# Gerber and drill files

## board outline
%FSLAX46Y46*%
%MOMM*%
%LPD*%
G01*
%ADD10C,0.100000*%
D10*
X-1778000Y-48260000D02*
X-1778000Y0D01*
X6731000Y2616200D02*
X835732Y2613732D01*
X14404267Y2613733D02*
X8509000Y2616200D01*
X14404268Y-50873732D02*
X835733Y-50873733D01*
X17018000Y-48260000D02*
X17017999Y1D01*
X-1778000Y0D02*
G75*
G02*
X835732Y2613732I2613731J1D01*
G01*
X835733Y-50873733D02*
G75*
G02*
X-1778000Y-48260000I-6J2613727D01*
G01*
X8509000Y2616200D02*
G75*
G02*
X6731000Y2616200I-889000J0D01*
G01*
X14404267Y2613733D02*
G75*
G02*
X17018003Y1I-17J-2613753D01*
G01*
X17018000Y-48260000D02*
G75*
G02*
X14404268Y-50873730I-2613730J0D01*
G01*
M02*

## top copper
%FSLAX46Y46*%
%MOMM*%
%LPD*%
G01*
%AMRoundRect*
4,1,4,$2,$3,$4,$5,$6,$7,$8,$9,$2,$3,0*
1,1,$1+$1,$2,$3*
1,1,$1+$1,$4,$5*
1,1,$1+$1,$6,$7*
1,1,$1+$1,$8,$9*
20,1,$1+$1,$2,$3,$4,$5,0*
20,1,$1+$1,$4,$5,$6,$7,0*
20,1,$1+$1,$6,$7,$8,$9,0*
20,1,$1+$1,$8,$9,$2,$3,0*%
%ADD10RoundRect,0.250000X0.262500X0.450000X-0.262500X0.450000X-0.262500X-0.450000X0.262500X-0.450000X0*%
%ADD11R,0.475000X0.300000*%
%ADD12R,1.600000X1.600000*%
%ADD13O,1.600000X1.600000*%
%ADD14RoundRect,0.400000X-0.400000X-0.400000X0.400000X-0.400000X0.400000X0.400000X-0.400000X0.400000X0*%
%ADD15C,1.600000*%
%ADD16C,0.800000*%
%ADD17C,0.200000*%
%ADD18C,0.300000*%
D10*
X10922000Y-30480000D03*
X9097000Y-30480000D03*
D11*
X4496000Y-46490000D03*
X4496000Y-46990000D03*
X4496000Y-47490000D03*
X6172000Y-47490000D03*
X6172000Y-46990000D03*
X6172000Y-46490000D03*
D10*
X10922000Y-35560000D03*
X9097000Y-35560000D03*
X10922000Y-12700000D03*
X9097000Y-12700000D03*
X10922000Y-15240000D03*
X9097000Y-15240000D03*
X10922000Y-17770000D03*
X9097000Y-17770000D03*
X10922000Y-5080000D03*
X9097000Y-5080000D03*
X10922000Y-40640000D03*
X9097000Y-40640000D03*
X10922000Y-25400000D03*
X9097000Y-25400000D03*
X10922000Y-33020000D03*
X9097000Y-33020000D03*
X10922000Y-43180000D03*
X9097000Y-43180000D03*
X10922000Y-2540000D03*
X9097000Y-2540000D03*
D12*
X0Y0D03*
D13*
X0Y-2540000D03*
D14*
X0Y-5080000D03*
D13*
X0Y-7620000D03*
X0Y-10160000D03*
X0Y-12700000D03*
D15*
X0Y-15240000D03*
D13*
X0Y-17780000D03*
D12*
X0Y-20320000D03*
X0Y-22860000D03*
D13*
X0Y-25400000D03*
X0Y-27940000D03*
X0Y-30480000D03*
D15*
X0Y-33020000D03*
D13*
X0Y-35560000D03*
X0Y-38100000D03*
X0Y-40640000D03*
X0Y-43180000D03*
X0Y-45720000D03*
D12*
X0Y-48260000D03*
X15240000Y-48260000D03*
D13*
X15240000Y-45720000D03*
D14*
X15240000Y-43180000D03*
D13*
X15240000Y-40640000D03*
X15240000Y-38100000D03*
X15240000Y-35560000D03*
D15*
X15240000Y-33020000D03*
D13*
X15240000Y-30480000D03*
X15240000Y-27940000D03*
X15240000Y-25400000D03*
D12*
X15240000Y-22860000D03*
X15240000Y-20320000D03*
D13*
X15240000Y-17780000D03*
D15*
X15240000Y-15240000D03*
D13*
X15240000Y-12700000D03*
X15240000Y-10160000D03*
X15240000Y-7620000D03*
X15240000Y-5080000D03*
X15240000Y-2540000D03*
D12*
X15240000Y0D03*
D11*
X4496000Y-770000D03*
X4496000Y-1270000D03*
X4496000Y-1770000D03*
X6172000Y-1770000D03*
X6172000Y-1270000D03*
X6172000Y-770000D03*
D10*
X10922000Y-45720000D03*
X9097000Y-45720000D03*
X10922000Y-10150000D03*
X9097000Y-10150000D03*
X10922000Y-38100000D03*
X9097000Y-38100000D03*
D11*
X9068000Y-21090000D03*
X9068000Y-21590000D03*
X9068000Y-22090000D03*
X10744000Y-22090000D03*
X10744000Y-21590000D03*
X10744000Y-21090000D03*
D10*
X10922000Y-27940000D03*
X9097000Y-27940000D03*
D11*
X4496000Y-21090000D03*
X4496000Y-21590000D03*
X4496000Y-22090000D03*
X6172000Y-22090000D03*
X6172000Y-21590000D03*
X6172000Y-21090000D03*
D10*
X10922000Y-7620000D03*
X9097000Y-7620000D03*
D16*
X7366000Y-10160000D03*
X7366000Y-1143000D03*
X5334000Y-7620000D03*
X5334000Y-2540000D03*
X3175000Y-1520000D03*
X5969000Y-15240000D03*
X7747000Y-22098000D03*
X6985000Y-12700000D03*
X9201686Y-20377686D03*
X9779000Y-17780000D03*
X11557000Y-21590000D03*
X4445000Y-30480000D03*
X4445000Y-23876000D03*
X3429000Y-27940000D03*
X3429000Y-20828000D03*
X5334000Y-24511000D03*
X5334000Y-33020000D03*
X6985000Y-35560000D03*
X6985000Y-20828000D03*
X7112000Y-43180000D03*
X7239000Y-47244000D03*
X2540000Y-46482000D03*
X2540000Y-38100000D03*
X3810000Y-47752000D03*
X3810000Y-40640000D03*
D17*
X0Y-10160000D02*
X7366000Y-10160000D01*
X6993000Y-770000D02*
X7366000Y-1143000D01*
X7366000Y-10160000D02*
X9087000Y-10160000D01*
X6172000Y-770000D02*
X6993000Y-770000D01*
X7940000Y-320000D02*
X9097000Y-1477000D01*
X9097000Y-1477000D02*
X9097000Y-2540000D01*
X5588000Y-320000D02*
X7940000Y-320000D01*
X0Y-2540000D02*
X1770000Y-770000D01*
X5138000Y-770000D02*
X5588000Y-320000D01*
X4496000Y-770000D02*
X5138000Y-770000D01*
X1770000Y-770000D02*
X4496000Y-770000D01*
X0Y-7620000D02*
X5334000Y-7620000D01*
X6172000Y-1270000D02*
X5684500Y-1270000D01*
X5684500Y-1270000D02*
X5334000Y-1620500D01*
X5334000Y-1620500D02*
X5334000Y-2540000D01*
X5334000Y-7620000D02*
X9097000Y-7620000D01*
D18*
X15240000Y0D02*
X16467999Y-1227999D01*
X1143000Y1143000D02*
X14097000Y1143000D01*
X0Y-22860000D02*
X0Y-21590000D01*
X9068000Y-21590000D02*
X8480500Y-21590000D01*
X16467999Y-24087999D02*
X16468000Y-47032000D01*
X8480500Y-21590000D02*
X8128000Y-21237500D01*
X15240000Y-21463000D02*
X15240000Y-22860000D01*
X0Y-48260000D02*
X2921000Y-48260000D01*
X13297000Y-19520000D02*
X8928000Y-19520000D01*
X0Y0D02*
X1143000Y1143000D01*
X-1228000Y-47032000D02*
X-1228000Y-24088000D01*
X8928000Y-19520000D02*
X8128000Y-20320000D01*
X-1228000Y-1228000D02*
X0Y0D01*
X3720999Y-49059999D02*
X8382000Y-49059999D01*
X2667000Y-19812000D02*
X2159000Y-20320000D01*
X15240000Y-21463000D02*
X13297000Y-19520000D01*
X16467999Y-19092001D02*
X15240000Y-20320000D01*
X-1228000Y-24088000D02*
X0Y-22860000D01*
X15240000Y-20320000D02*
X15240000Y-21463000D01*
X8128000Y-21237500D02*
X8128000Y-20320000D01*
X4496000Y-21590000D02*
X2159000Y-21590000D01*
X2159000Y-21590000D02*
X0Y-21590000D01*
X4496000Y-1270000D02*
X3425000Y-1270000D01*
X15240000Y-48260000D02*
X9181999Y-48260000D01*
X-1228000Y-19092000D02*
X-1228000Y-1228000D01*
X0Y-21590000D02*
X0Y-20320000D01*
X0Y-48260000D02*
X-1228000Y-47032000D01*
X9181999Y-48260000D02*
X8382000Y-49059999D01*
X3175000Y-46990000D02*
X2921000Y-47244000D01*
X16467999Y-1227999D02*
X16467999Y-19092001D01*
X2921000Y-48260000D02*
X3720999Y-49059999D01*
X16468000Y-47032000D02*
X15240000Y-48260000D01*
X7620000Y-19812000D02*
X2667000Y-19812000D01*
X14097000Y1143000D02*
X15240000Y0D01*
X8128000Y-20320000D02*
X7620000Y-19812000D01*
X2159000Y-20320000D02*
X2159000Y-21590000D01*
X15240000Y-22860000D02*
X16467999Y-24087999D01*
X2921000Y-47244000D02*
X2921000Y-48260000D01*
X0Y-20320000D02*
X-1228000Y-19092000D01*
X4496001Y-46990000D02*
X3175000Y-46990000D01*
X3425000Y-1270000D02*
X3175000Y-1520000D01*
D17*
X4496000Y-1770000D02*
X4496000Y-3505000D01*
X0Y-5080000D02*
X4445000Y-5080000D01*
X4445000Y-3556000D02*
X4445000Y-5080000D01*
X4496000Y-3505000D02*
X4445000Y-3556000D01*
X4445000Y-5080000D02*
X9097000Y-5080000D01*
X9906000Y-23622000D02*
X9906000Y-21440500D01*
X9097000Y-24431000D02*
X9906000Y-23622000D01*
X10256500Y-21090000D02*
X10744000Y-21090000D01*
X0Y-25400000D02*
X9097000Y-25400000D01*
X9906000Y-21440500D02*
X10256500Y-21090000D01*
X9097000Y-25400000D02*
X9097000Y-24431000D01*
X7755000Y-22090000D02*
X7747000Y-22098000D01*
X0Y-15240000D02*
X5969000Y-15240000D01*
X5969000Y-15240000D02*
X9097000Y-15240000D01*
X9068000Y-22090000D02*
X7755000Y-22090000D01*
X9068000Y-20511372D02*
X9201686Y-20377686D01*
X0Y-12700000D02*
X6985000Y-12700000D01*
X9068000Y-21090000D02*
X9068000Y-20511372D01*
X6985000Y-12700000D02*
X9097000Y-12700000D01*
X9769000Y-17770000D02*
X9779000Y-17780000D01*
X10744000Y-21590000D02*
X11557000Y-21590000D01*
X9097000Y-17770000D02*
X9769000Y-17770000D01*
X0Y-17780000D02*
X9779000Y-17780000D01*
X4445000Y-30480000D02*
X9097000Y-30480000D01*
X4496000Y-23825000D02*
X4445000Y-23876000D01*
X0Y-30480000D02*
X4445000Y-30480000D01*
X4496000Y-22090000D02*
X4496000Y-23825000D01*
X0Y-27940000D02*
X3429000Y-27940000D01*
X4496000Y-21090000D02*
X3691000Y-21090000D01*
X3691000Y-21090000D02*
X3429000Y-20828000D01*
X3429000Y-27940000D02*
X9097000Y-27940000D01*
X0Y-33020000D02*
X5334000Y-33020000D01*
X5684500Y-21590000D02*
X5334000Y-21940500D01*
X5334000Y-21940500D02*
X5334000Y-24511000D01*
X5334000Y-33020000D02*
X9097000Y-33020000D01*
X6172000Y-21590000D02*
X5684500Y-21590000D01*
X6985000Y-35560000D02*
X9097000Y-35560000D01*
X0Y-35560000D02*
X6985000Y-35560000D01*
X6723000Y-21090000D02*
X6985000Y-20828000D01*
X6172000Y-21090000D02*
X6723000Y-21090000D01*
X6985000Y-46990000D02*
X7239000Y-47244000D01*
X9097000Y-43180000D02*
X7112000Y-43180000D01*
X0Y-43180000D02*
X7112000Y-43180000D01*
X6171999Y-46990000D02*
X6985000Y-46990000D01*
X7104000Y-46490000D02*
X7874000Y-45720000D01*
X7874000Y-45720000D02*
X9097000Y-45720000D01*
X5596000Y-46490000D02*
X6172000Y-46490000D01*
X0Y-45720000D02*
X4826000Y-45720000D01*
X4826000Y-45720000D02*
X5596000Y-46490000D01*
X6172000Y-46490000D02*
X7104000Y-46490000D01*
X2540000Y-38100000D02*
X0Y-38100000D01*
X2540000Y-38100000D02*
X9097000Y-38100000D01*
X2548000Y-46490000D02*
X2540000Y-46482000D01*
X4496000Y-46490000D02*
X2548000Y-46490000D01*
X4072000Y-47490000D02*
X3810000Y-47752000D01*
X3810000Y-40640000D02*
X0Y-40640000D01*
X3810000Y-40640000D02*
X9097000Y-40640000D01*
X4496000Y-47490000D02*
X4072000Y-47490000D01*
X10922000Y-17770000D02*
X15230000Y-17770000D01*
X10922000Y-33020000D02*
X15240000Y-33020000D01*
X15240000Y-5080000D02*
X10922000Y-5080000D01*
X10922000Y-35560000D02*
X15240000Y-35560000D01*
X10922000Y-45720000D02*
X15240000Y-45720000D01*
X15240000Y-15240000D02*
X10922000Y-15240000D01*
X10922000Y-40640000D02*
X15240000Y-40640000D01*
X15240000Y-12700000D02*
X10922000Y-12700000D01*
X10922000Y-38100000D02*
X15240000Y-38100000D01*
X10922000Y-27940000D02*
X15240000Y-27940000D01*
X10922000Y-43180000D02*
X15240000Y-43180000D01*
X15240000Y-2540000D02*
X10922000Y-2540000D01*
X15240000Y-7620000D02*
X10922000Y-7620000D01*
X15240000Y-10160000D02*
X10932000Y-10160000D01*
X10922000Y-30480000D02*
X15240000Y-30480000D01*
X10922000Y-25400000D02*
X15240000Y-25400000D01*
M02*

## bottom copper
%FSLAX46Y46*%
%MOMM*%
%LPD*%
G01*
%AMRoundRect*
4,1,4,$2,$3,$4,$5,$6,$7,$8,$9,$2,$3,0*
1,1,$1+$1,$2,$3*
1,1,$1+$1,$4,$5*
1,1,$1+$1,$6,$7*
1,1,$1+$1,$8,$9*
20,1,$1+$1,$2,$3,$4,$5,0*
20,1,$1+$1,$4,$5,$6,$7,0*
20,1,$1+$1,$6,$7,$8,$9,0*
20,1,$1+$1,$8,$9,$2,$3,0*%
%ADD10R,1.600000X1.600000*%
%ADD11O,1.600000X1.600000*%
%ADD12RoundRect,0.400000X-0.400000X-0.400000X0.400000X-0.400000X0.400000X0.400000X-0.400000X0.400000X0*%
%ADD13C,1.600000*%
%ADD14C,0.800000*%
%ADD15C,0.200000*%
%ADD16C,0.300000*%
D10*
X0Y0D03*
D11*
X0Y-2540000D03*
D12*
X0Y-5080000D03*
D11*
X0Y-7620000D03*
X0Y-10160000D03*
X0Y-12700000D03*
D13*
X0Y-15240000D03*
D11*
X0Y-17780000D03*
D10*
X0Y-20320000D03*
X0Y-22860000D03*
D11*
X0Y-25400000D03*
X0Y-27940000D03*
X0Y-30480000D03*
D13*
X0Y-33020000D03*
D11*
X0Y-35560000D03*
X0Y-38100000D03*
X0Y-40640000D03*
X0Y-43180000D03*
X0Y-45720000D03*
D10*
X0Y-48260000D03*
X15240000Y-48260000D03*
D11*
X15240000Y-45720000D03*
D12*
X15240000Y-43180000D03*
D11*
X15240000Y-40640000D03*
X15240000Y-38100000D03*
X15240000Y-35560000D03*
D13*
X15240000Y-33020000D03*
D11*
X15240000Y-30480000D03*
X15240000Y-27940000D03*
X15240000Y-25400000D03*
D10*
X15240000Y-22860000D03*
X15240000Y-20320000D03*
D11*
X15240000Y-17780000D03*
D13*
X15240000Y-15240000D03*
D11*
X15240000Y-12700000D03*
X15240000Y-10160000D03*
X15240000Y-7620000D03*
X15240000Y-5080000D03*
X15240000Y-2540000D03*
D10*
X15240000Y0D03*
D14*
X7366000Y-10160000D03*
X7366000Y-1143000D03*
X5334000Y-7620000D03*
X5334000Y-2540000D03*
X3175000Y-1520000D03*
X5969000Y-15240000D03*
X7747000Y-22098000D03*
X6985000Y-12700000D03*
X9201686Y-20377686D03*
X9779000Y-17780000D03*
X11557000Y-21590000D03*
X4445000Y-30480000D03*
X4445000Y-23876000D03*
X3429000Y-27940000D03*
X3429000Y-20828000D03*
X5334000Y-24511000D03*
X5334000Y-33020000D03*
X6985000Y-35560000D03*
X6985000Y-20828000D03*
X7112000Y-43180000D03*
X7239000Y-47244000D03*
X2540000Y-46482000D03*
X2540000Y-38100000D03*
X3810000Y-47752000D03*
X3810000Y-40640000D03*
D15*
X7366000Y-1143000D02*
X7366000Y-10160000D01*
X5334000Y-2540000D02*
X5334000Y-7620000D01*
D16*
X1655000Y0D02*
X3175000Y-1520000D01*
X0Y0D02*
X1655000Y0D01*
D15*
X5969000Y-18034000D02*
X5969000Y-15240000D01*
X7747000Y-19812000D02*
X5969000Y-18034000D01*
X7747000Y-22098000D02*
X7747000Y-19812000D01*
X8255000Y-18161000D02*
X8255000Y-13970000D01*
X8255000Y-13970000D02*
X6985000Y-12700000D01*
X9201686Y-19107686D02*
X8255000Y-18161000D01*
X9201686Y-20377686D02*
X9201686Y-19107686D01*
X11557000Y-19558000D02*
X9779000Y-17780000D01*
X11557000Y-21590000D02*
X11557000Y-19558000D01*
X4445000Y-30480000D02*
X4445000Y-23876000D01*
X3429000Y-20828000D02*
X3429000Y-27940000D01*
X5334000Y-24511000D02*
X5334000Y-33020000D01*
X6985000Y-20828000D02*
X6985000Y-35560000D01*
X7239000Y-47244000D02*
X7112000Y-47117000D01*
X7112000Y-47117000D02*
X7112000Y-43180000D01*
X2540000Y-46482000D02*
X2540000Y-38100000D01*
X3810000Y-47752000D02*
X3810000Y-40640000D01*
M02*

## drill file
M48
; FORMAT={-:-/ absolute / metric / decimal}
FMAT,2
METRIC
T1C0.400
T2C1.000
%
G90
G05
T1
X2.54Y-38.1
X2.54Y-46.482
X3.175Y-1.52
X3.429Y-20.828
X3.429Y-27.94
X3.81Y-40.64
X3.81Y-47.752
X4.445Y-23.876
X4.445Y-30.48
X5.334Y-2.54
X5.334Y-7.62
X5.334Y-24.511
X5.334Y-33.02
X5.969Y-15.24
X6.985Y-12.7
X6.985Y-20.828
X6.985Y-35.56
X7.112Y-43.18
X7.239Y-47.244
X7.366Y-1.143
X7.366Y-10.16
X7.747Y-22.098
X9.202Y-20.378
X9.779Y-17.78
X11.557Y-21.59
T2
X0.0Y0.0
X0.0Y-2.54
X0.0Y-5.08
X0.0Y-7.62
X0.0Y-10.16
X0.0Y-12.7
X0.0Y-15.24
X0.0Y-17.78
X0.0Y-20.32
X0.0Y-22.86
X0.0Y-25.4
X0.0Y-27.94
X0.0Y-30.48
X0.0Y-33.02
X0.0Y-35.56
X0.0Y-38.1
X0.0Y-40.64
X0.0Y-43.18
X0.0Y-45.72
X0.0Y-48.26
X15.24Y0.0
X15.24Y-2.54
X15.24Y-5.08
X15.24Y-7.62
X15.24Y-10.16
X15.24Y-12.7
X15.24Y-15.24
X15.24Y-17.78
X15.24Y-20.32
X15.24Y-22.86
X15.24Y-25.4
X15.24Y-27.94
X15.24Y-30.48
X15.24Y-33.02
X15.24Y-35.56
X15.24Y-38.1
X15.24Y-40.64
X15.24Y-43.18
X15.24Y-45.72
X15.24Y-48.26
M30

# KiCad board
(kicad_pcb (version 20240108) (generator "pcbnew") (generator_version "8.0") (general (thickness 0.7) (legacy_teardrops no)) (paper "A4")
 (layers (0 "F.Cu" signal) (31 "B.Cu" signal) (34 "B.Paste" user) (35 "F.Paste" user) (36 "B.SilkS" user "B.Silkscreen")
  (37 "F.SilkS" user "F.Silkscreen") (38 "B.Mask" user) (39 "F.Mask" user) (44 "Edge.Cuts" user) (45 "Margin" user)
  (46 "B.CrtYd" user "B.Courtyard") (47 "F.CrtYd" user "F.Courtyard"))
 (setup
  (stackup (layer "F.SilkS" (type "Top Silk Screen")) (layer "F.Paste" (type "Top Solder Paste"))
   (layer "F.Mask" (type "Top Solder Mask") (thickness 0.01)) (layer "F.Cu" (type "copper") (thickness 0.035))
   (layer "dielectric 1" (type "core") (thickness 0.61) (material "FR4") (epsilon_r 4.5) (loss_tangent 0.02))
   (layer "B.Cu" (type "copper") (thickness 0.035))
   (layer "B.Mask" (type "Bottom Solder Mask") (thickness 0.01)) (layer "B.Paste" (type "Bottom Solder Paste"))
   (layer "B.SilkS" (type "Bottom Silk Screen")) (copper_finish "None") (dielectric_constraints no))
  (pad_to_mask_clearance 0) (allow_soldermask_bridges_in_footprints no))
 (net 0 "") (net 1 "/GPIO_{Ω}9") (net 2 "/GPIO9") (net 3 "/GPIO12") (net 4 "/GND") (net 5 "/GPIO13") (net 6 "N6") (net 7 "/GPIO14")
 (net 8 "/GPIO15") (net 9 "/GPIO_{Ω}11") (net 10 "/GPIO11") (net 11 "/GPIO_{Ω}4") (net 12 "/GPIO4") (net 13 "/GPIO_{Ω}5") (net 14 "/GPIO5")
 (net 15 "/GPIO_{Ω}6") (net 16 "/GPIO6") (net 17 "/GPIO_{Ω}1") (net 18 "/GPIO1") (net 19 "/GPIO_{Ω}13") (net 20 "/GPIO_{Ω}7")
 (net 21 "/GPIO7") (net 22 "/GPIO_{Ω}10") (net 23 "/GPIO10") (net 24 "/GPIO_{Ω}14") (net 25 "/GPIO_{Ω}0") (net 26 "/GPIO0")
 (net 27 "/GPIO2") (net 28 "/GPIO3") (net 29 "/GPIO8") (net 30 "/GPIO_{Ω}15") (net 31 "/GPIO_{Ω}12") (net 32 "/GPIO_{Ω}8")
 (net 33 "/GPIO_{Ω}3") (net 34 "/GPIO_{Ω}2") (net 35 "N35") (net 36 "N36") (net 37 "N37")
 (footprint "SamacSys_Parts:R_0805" (layer "F.Cu") (at 10.0095 30.47 90)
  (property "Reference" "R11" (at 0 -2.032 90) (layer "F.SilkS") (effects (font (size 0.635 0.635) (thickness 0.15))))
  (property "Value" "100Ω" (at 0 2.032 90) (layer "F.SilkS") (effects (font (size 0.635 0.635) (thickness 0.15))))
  (pad "1" smd roundrect (at -0.01 0.9125 180) (size 1.025 1.4) (layers "F.Cu" "F.Paste" "F.Mask") (roundrect_rratio 0.243902)
   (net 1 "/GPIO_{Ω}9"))
  (pad "2" smd roundrect (at -0.01 -0.9125 180) (size 1.025 1.4) (layers "F.Cu" "F.Paste" "F.Mask") (roundrect_rratio 0.243902)
   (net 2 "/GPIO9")))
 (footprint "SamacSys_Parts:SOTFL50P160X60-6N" (layer "F.Cu") (at 5.334 46.99)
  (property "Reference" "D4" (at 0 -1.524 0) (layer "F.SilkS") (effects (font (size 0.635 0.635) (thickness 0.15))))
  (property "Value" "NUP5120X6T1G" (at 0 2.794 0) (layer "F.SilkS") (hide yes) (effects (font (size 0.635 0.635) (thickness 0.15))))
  (pad "1" smd rect (at -0.838 -0.5 90) (size 0.3 0.475) (layers "F.Cu" "F.Paste" "F.Mask") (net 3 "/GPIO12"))
  (pad "2" smd rect (at -0.838 0 90) (size 0.3 0.475) (layers "F.Cu" "F.Paste" "F.Mask") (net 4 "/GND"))
  (pad "3" smd rect (at -0.838 0.5 90) (size 0.3 0.475) (layers "F.Cu" "F.Paste" "F.Mask") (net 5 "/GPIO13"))
  (pad "4" smd rect (at 0.838 0.5 90) (size 0.3 0.475) (layers "F.Cu" "F.Paste" "F.Mask") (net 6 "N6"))
  (pad "5" smd rect (at 0.838 0 90) (size 0.3 0.475) (layers "F.Cu" "F.Paste" "F.Mask") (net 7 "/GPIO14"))
  (pad "6" smd rect (at 0.838 -0.5 90) (size 0.3 0.475) (layers "F.Cu" "F.Paste" "F.Mask") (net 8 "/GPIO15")))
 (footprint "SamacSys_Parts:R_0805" (layer "F.Cu") (at 10.0095 35.55 90)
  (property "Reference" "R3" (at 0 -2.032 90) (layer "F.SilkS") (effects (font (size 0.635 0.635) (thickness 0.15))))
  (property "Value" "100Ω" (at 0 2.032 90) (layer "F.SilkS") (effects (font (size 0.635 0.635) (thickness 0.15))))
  (pad "1" smd roundrect (at -0.01 0.9125 180) (size 1.025 1.4) (layers "F.Cu" "F.Paste" "F.Mask") (roundrect_rratio 0.243902)
   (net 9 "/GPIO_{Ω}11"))
  (pad "2" smd roundrect (at -0.01 -0.9125 180) (size 1.025 1.4) (layers "F.Cu" "F.Paste" "F.Mask") (roundrect_rratio 0.243902)
   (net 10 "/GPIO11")))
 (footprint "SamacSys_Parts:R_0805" (layer "F.Cu") (at 10.0095 12.69 90)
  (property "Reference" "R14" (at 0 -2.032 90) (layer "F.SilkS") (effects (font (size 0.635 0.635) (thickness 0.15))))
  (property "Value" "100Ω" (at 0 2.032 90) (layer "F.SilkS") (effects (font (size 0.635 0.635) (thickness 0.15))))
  (pad "1" smd roundrect (at -0.01 0.9125 180) (size 1.025 1.4) (layers "F.Cu" "F.Paste" "F.Mask") (roundrect_rratio 0.243902)
   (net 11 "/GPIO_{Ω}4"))
  (pad "2" smd roundrect (at -0.01 -0.9125 180) (size 1.025 1.4) (layers "F.Cu" "F.Paste" "F.Mask") (roundrect_rratio 0.243902)
   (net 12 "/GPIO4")))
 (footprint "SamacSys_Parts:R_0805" (layer "F.Cu") (at 10.0095 15.23 90)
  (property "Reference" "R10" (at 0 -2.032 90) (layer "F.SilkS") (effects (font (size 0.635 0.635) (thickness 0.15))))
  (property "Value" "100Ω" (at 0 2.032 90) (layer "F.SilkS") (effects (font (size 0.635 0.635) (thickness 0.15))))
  (pad "1" smd roundrect (at -0.01 0.9125 180) (size 1.025 1.4) (layers "F.Cu" "F.Paste" "F.Mask") (roundrect_rratio 0.243902)
   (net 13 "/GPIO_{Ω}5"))
  (pad "2" smd roundrect (at -0.01 -0.9125 180) (size 1.025 1.4) (layers "F.Cu" "F.Paste" "F.Mask") (roundrect_rratio 0.243902)
   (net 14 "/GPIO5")))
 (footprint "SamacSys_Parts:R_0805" (layer "F.Cu") (at 10.0095 17.76 90)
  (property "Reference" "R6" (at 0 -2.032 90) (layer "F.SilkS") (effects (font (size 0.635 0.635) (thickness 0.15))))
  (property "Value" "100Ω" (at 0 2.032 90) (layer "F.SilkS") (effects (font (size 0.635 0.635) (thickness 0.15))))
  (pad "1" smd roundrect (at -0.01 0.9125 180) (size 1.025 1.4) (layers "F.Cu" "F.Paste" "F.Mask") (roundrect_rratio 0.243902)
   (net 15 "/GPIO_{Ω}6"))
  (pad "2" smd roundrect (at -0.01 -0.9125 180) (size 1.025 1.4) (layers "F.Cu" "F.Paste" "F.Mask") (roundrect_rratio 0.243902)
   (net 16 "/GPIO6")))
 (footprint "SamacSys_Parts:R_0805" (layer "F.Cu") (at 10.0095 5.07 90)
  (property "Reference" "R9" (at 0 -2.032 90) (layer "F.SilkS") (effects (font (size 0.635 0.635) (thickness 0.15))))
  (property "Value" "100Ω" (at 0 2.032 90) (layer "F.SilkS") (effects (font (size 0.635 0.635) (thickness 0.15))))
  (pad "1" smd roundrect (at -0.01 0.9125 180) (size 1.025 1.4) (layers "F.Cu" "F.Paste" "F.Mask") (roundrect_rratio 0.243902)
   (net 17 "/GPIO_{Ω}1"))
  (pad "2" smd roundrect (at -0.01 -0.9125 180) (size 1.025 1.4) (layers "F.Cu" "F.Paste" "F.Mask") (roundrect_rratio 0.243902)
   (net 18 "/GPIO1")))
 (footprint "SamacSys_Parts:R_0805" (layer "F.Cu") (at 10.0095 40.63 90)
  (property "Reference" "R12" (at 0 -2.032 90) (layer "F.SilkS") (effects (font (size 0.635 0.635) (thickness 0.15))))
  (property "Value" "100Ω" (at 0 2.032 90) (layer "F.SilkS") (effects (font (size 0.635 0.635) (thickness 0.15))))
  (pad "1" smd roundrect (at -0.01 0.9125 180) (size 1.025 1.4) (layers "F.Cu" "F.Paste" "F.Mask") (roundrect_rratio 0.243902)
   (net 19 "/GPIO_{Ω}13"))
  (pad "2" smd roundrect (at -0.01 -0.9125 180) (size 1.025 1.4) (layers "F.Cu" "F.Paste" "F.Mask") (roundrect_rratio 0.243902)
   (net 5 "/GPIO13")))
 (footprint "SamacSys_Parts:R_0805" (layer "F.Cu") (at 10.0095 25.39 90)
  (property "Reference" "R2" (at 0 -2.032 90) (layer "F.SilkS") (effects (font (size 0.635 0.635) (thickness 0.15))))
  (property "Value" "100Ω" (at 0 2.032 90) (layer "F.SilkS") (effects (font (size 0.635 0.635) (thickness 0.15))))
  (pad "1" smd roundrect (at -0.01 0.9125 180) (size 1.025 1.4) (layers "F.Cu" "F.Paste" "F.Mask") (roundrect_rratio 0.243902)
   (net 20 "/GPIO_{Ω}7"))
  (pad "2" smd roundrect (at -0.01 -0.9125 180) (size 1.025 1.4) (layers "F.Cu" "F.Paste" "F.Mask") (roundrect_rratio 0.243902)
   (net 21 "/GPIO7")))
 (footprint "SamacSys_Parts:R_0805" (layer "F.Cu") (at 10.0095 33.01 90)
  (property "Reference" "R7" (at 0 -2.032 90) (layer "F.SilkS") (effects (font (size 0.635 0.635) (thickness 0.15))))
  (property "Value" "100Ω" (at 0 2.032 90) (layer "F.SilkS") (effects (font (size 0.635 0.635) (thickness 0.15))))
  (pad "1" smd roundrect (at -0.01 0.9125 180) (size 1.025 1.4) (layers "F.Cu" "F.Paste" "F.Mask") (roundrect_rratio 0.243902)
   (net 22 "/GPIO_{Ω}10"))
  (pad "2" smd roundrect (at -0.01 -0.9125 180) (size 1.025 1.4) (layers "F.Cu" "F.Paste" "F.Mask") (roundrect_rratio 0.243902)
   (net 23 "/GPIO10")))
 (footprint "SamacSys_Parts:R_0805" (layer "F.Cu") (at 10.0095 43.17 90)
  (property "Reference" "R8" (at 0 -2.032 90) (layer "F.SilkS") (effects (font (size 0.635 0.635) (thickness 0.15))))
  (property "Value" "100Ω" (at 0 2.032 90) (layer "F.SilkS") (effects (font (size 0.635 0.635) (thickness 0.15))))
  (pad "1" smd roundrect (at -0.01 0.9125 180) (size 1.025 1.4) (layers "F.Cu" "F.Paste" "F.Mask") (roundrect_rratio 0.243902)
   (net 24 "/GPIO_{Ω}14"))
  (pad "2" smd roundrect (at -0.01 -0.9125 180) (size 1.025 1.4) (layers "F.Cu" "F.Paste" "F.Mask") (roundrect_rratio 0.243902)
   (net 7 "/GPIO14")))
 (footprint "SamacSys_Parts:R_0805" (layer "F.Cu") (at 10.0095 2.53 90)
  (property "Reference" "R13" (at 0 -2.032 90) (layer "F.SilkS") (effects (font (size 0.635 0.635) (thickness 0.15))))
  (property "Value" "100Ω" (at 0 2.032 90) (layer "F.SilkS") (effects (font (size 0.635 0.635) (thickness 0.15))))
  (pad "1" smd roundrect (at -0.01 0.9125 180) (size 1.025 1.4) (layers "F.Cu" "F.Paste" "F.Mask") (roundrect_rratio 0.243902)
   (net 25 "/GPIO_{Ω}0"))
  (pad "2" smd roundrect (at -0.01 -0.9125 180) (size 1.025 1.4) (layers "F.Cu" "F.Paste" "F.Mask") (roundrect_rratio 0.243902)
   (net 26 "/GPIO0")))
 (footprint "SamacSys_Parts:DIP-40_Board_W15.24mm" (layer "F.Cu") (at 0 0)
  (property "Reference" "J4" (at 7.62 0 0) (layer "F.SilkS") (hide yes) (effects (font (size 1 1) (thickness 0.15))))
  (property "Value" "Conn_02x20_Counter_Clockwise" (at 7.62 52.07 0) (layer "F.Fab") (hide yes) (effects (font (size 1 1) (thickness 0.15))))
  (fp_line (start -1.778 48.26) (end -1.778 0) (stroke (width 0.1) (type solid)) (layer "Edge.Cuts"))
  (fp_line (start 6.731 -2.6162) (end 0.835732 -2.613732) (stroke (width 0.1) (type solid)) (layer "Edge.Cuts"))
  (fp_line (start 14.404267 -2.613733) (end 8.509 -2.6162) (stroke (width 0.1) (type solid)) (layer "Edge.Cuts"))
  (fp_line (start 14.404268 50.873732) (end 0.835733 50.873733) (stroke (width 0.1) (type solid)) (layer "Edge.Cuts"))
  (fp_line (start 17.018 48.26) (end 17.017999 -0.000001) (stroke (width 0.1) (type solid)) (layer "Edge.Cuts"))
  (fp_arc (start -1.778 0) (mid -1.012456 -1.848188) (end 0.835732 -2.613732) (stroke (width 0.1) (type solid)) (layer "Edge.Cuts"))
  (fp_arc (start 0.835733 50.873733) (mid -1.012457 50.10819) (end -1.778 48.26) (stroke (width 0.1) (type solid)) (layer "Edge.Cuts"))
  (fp_arc (start 8.509 -2.6162) (mid 7.62 -1.7272) (end 6.731 -2.6162) (stroke (width 0.1) (type default)) (layer "Edge.Cuts"))
  (fp_arc (start 14.404267 -2.613733) (mid 16.252448 -1.848183) (end 17.017999 -0.000001) (stroke (width 0.1) (type solid))
   (layer "Edge.Cuts"))
  (fp_arc (start 17.018 48.26) (mid 16.252456 50.108187) (end 14.404268 50.873732) (stroke (width 0.1) (type solid)) (layer "Edge.Cuts"))
  (pad "1" thru_hole rect (at 0 0) (size 1.6 1.6) (drill 1) (layers "*.Cu" "*.Mask") (remove_unused_layers no) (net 4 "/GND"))
  (pad "2" thru_hole oval (at 0 2.54) (size 1.6 1.6) (drill 1) (layers "*.Cu" "*.Mask") (remove_unused_layers no) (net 26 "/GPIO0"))
  (pad "3" thru_hole roundrect (at 0 5.08) (size 1.6 1.6) (drill 1) (layers "*.Cu" "*.Mask") (remove_unused_layers no)
   (roundrect_rratio 0.25) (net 18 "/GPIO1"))
  (pad "4" thru_hole oval (at 0 7.62) (size 1.6 1.6) (drill 1) (layers "*.Cu" "*.Mask") (remove_unused_layers no) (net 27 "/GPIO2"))
  (pad "5" thru_hole oval (at 0 10.16) (size 1.6 1.6) (drill 1) (layers "*.Cu" "*.Mask") (remove_unused_layers no) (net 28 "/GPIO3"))
  (pad "6" thru_hole oval (at 0 12.7) (size 1.6 1.6) (drill 1) (layers "*.Cu" "*.Mask") (remove_unused_layers no) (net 12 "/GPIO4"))
  (pad "7" thru_hole circle (at 0 15.24) (size 1.6 1.6) (drill 1) (layers "*.Cu" "*.Mask") (remove_unused_layers no) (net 14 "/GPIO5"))
  (pad "8" thru_hole oval (at 0 17.78) (size 1.6 1.6) (drill 1) (layers "*.Cu" "*.Mask") (remove_unused_layers no) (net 16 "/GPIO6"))
  (pad "9" thru_hole rect (at 0 20.32) (size 1.6 1.6) (drill 1) (layers "*.Cu" "*.Mask") (remove_unused_layers no) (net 4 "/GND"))
  (pad "10" thru_hole rect (at 0 22.86) (size 1.6 1.6) (drill 1) (layers "*.Cu" "*.Mask") (remove_unused_layers no) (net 4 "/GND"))
  (pad "11" thru_hole oval (at 0 25.4) (size 1.6 1.6) (drill 1) (layers "*.Cu" "*.Mask") (remove_unused_layers no) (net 21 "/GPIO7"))
  (pad "12" thru_hole oval (at 0 27.94) (size 1.6 1.6) (drill 1) (layers "*.Cu" "*.Mask") (remove_unused_layers no) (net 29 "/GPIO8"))
  (pad "13" thru_hole oval (at 0 30.48) (size 1.6 1.6) (drill 1) (layers "*.Cu" "*.Mask") (remove_unused_layers no) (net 2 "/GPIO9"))
  (pad "14" thru_hole circle (at 0 33.02) (size 1.6 1.6) (drill 1) (layers "*.Cu" "*.Mask") (remove_unused_layers no) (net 23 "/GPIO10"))
  (pad "15" thru_hole oval (at 0 35.56) (size 1.6 1.6) (drill 1) (layers "*.Cu" "*.Mask") (remove_unused_layers no) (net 10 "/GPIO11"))
  (pad "16" thru_hole oval (at 0 38.1) (size 1.6 1.6) (drill 1) (layers "*.Cu" "*.Mask") (remove_unused_layers no) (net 3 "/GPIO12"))
  (pad "17" thru_hole oval (at 0 40.64) (size 1.6 1.6) (drill 1) (layers "*.Cu" "*.Mask") (remove_unused_layers no) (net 5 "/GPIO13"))
  (pad "18" thru_hole oval (at 0 43.18) (size 1.6 1.6) (drill 1) (layers "*.Cu" "*.Mask") (remove_unused_layers no) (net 7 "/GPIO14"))
  (pad "19" thru_hole oval (at 0 45.72) (size 1.6 1.6) (drill 1) (layers "*.Cu" "*.Mask") (remove_unused_layers no) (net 8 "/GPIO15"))
  (pad "20" thru_hole rect (at 0 48.26) (size 1.6 1.6) (drill 1) (layers "*.Cu" "*.Mask") (remove_unused_layers no) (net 4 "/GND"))
  (pad "21" thru_hole rect (at 15.24 48.26) (size 1.6 1.6) (drill 1) (layers "*.Cu" "*.Mask") (remove_unused_layers no) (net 4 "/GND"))
  (pad "22" thru_hole oval (at 15.24 45.72) (size 1.6 1.6) (drill 1) (layers "*.Cu" "*.Mask") (remove_unused_layers no)
   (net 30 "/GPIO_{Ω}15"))
  (pad "23" thru_hole roundrect (at 15.24 43.18) (size 1.6 1.6) (drill 1) (layers "*.Cu" "*.Mask") (remove_unused_layers no)
   (roundrect_rratio 0.25) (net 24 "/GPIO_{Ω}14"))
  (pad "24" thru_hole oval (at 15.24 40.64) (size 1.6 1.6) (drill 1) (layers "*.Cu" "*.Mask") (remove_unused_layers no)
   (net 19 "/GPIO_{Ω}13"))
  (pad "25" thru_hole oval (at 15.24 38.1) (size 1.6 1.6) (drill 1) (layers "*.Cu" "*.Mask") (remove_unused_layers no)
   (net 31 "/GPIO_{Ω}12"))
  (pad "26" thru_hole oval (at 15.24 35.56) (size 1.6 1.6) (drill 1) (layers "*.Cu" "*.Mask") (remove_unused_layers no)
   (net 9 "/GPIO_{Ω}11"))
  (pad "27" thru_hole circle (at 15.24 33.02) (size 1.6 1.6) (drill 1) (layers "*.Cu" "*.Mask") (remove_unused_layers no)
   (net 22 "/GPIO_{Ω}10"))
  (pad "28" thru_hole oval (at 15.24 30.48) (size 1.6 1.6) (drill 1) (layers "*.Cu" "*.Mask") (remove_unused_layers no) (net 1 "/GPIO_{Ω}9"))
  (pad "29" thru_hole oval (at 15.24 27.94) (size 1.6 1.6) (drill 1) (layers "*.Cu" "*.Mask") (remove_unused_layers no)
   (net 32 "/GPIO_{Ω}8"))
  (pad "30" thru_hole oval (at 15.24 25.4) (size 1.6 1.6) (drill 1) (layers "*.Cu" "*.Mask") (remove_unused_layers no) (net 20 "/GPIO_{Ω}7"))
  (pad "31" thru_hole rect (at 15.24 22.86) (size 1.6 1.6) (drill 1) (layers "*.Cu" "*.Mask") (remove_unused_layers no) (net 4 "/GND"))
  (pad "32" thru_hole rect (at 15.24 20.32) (size 1.6 1.6) (drill 1) (layers "*.Cu" "*.Mask") (remove_unused_layers no) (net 4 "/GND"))
  (pad "33" thru_hole oval (at 15.24 17.78) (size 1.6 1.6) (drill 1) (layers "*.Cu" "*.Mask") (remove_unused_layers no)
   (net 15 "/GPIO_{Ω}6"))
  (pad "34" thru_hole circle (at 15.24 15.24) (size 1.6 1.6) (drill 1) (layers "*.Cu" "*.Mask") (remove_unused_layers no)
   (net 13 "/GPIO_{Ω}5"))
  (pad "35" thru_hole oval (at 15.24 12.7) (size 1.6 1.6) (drill 1) (layers "*.Cu" "*.Mask") (remove_unused_layers no) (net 11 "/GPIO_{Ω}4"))
  (pad "36" thru_hole oval (at 15.24 10.16) (size 1.6 1.6) (drill 1) (layers "*.Cu" "*.Mask") (remove_unused_layers no)
   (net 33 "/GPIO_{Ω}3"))
  (pad "37" thru_hole oval (at 15.24 7.62) (size 1.6 1.6) (drill 1) (layers "*.Cu" "*.Mask") (remove_unused_layers no) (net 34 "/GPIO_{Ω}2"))
  (pad "38" thru_hole oval (at 15.24 5.08) (size 1.6 1.6) (drill 1) (layers "*.Cu" "*.Mask") (remove_unused_layers no) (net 17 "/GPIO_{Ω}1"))
  (pad "39" thru_hole oval (at 15.24 2.54) (size 1.6 1.6) (drill 1) (layers "*.Cu" "*.Mask") (remove_unused_layers no) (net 25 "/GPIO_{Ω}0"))
  (pad "40" thru_hole rect (at 15.24 0) (size 1.6 1.6) (drill 1) (layers "*.Cu" "*.Mask") (remove_unused_layers no) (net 4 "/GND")))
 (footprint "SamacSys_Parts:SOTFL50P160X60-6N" (layer "F.Cu") (at 5.334 1.27)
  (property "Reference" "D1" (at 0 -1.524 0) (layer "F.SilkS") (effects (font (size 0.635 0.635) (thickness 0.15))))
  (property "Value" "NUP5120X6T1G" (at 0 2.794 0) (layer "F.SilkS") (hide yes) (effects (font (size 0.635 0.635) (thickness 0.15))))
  (pad "1" smd rect (at -0.838 -0.5 90) (size 0.3 0.475) (layers "F.Cu" "F.Paste" "F.Mask") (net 26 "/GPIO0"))
  (pad "2" smd rect (at -0.838 0 90) (size 0.3 0.475) (layers "F.Cu" "F.Paste" "F.Mask") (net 4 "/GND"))
  (pad "3" smd rect (at -0.838 0.5 90) (size 0.3 0.475) (layers "F.Cu" "F.Paste" "F.Mask") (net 18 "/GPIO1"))
  (pad "4" smd rect (at 0.838 0.5 90) (size 0.3 0.475) (layers "F.Cu" "F.Paste" "F.Mask") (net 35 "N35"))
  (pad "5" smd rect (at 0.838 0 90) (size 0.3 0.475) (layers "F.Cu" "F.Paste" "F.Mask") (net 27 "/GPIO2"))
  (pad "6" smd rect (at 0.838 -0.5 90) (size 0.3 0.475) (layers "F.Cu" "F.Paste" "F.Mask") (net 28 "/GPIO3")))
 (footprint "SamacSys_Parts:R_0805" (layer "F.Cu") (at 10.0095 45.71 90)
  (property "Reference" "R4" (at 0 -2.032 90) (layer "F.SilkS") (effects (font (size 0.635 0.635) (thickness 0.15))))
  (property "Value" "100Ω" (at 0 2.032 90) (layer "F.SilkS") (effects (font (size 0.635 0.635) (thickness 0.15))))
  (pad "1" smd roundrect (at -0.01 0.9125 180) (size 1.025 1.4) (layers "F.Cu" "F.Paste" "F.Mask") (roundrect_rratio 0.243902)
   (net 30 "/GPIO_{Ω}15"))
  (pad "2" smd roundrect (at -0.01 -0.9125 180) (size 1.025 1.4) (layers "F.Cu" "F.Paste" "F.Mask") (roundrect_rratio 0.243902)
   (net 8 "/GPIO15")))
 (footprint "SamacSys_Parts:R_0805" (layer "F.Cu") (at 10.0095 10.14 90)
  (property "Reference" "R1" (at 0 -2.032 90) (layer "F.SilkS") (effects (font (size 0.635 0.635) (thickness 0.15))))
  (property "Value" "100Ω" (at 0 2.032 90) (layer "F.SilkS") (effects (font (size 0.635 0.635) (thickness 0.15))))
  (pad "1" smd roundrect (at -0.01 0.9125 180) (size 1.025 1.4) (layers "F.Cu" "F.Paste" "F.Mask") (roundrect_rratio 0.243902)
   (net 33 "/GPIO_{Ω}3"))
  (pad "2" smd roundrect (at -0.01 -0.9125 180) (size 1.025 1.4) (layers "F.Cu" "F.Paste" "F.Mask") (roundrect_rratio 0.243902)
   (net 28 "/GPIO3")))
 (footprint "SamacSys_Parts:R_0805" (layer "F.Cu") (at 10.0095 38.09 90)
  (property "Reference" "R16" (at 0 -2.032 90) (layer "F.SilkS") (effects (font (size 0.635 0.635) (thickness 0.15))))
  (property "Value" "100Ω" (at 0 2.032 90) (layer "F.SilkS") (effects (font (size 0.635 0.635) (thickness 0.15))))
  (pad "1" smd roundrect (at -0.01 0.9125 180) (size 1.025 1.4) (layers "F.Cu" "F.Paste" "F.Mask") (roundrect_rratio 0.243902)
   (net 31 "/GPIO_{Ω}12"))
  (pad "2" smd roundrect (at -0.01 -0.9125 180) (size 1.025 1.4) (layers "F.Cu" "F.Paste" "F.Mask") (roundrect_rratio 0.243902)
   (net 3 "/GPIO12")))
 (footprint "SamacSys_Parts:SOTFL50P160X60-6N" (layer "F.Cu") (at 9.906 21.59)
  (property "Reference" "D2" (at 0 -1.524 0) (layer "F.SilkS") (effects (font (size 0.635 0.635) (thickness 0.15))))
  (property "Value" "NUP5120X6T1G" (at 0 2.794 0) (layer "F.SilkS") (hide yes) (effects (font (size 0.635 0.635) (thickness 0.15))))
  (pad "1" smd rect (at -0.838 -0.5 90) (size 0.3 0.475) (layers "F.Cu" "F.Paste" "F.Mask") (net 12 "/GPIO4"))
  (pad "2" smd rect (at -0.838 0 90) (size 0.3 0.475) (layers "F.Cu" "F.Paste" "F.Mask") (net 4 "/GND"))
  (pad "3" smd rect (at -0.838 0.5 90) (size 0.3 0.475) (layers "F.Cu" "F.Paste" "F.Mask") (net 14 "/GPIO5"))
  (pad "4" smd rect (at 0.838 0.5 90) (size 0.3 0.475) (layers "F.Cu" "F.Paste" "F.Mask") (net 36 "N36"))
  (pad "5" smd rect (at 0.838 0 90) (size 0.3 0.475) (layers "F.Cu" "F.Paste" "F.Mask") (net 16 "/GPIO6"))
  (pad "6" smd rect (at 0.838 -0.5 90) (size 0.3 0.475) (layers "F.Cu" "F.Paste" "F.Mask") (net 21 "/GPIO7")))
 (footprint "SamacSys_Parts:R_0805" (layer "F.Cu") (at 10.0095 27.93 90)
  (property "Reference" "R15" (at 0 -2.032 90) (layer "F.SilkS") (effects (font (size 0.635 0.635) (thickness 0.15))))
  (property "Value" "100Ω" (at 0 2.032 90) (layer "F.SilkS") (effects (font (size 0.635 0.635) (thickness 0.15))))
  (pad "1" smd roundrect (at -0.01 0.9125 180) (size 1.025 1.4) (layers "F.Cu" "F.Paste" "F.Mask") (roundrect_rratio 0.243902)
   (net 32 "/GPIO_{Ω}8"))
  (pad "2" smd roundrect (at -0.01 -0.9125 180) (size 1.025 1.4) (layers "F.Cu" "F.Paste" "F.Mask") (roundrect_rratio 0.243902)
   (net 29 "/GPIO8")))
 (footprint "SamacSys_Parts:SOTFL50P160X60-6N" (layer "F.Cu") (at 5.334 21.59)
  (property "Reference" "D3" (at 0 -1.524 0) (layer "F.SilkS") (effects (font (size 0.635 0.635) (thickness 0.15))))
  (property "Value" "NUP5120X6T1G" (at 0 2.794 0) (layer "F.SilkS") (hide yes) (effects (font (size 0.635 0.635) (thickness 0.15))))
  (pad "1" smd rect (at -0.838 -0.5 90) (size 0.3 0.475) (layers "F.Cu" "F.Paste" "F.Mask") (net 29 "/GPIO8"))
  (pad "2" smd rect (at -0.838 0 90) (size 0.3 0.475) (layers "F.Cu" "F.Paste" "F.Mask") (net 4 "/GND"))
  (pad "3" smd rect (at -0.838 0.5 90) (size 0.3 0.475) (layers "F.Cu" "F.Paste" "F.Mask") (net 2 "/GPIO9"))
  (pad "4" smd rect (at 0.838 0.5 90) (size 0.3 0.475) (layers "F.Cu" "F.Paste" "F.Mask") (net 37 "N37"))
  (pad "5" smd rect (at 0.838 0 90) (size 0.3 0.475) (layers "F.Cu" "F.Paste" "F.Mask") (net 23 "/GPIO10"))
  (pad "6" smd rect (at 0.838 -0.5 90) (size 0.3 0.475) (layers "F.Cu" "F.Paste" "F.Mask") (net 10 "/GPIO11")))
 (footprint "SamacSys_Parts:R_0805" (layer "F.Cu") (at 10.0095 7.61 90)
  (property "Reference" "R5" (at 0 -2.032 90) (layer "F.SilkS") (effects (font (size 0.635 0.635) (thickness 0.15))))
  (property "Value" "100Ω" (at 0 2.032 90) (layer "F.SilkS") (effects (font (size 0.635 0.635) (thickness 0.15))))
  (pad "1" smd roundrect (at -0.01 0.9125 180) (size 1.025 1.4) (layers "F.Cu" "F.Paste" "F.Mask") (roundrect_rratio 0.243902)
   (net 34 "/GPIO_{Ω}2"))
  (pad "2" smd roundrect (at -0.01 -0.9125 180) (size 1.025 1.4) (layers "F.Cu" "F.Paste" "F.Mask") (roundrect_rratio 0.243902)
   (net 27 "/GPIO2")))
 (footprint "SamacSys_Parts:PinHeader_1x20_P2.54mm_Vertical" (layer "B.Cu") (at 15.24 0 180)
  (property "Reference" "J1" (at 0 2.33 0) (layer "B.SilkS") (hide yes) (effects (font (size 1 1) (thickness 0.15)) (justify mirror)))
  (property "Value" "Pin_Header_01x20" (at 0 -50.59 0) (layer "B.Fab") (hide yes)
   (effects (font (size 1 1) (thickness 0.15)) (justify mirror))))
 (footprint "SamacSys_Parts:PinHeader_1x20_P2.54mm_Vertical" (layer "B.Cu") (at 0 0 180)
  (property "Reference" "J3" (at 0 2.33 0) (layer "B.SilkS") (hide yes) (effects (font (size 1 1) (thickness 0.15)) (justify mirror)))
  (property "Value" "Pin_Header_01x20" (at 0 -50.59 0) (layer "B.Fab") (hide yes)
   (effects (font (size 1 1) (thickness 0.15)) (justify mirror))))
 (segment (start 0 10.16) (end 7.366 10.16) (width 0.2) (layer "F.Cu") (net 28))
 (segment (start 6.993 0.77) (end 7.366 1.143) (width 0.2) (layer "F.Cu") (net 28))
 (segment (start 7.366 10.16) (end 9.087 10.16) (width 0.2) (layer "F.Cu") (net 28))
 (segment (start 6.172 0.77) (end 6.993 0.77) (width 0.2) (layer "F.Cu") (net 28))
 (via (at 7.366 10.16) (size 0.8) (drill 0.4) (layers "F.Cu" "B.Cu") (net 28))
 (via (at 7.366 1.143) (size 0.8) (drill 0.4) (layers "F.Cu" "B.Cu") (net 28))
 (segment (start 7.366 1.143) (end 7.366 10.16) (width 0.2) (layer "B.Cu") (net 28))
 (segment (start 7.94 0.32) (end 9.097 1.477) (width 0.2) (layer "F.Cu") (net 26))
 (segment (start 9.097 1.477) (end 9.097 2.54) (width 0.2) (layer "F.Cu") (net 26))
 (segment (start 5.588 0.32) (end 7.94 0.32) (width 0.2) (layer "F.Cu") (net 26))
 (segment (start 0 2.54) (end 1.77 0.77) (width 0.2) (layer "F.Cu") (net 26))
 (segment (start 5.138 0.77) (end 5.588 0.32) (width 0.2) (layer "F.Cu") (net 26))
 (segment (start 4.496 0.77) (end 5.138 0.77) (width 0.2) (layer "F.Cu") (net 26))
 (segment (start 1.77 0.77) (end 4.496 0.77) (width 0.2) (layer "F.Cu") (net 26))
 (segment (start 0 7.62) (end 5.334 7.62) (width 0.2) (layer "F.Cu") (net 27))
 (segment (start 6.172 1.27) (end 5.6845 1.27) (width 0.2) (layer "F.Cu") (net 27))
 (segment (start 5.6845 1.27) (end 5.334 1.6205) (width 0.2) (layer "F.Cu") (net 27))
 (segment (start 5.334 1.6205) (end 5.334 2.54) (width 0.2) (layer "F.Cu") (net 27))
 (segment (start 5.334 7.62) (end 9.097 7.62) (width 0.2) (layer "F.Cu") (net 27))
 (via (at 5.334 7.62) (size 0.8) (drill 0.4) (layers "F.Cu" "B.Cu") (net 27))
 (via (at 5.334 2.54) (size 0.8) (drill 0.4) (layers "F.Cu" "B.Cu") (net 27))
 (segment (start 5.334 2.54) (end 5.334 7.62) (width 0.2) (layer "B.Cu") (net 27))
 (segment (start 15.24 0) (end 16.467999 1.227999) (width 0.3) (layer "F.Cu") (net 4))
 (segment (start 1.143 -1.143) (end 14.097 -1.143) (width 0.3) (layer "F.Cu") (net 4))
 (segment (start 0 22.86) (end 0 21.59) (width 0.3) (layer "F.Cu") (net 4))
 (segment (start 9.068 21.59) (end 8.4805 21.59) (width 0.3) (layer "F.Cu") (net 4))
 (segment (start 16.467999 24.087999) (end 16.468 47.032) (width 0.3) (layer "F.Cu") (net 4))
 (segment (start 8.4805 21.59) (end 8.128 21.2375) (width 0.3) (layer "F.Cu") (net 4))
 (segment (start 15.24 21.463) (end 15.24 22.86) (width 0.3) (layer "F.Cu") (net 4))
 (segment (start 0 48.26) (end 2.921 48.26) (width 0.3) (layer "F.Cu") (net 4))
 (segment (start 13.297 19.52) (end 8.928 19.52) (width 0.3) (layer "F.Cu") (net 4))
 (segment (start 0 0) (end 1.143 -1.143) (width 0.3) (layer "F.Cu") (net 4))
 (segment (start -1.228 47.032) (end -1.228 24.088) (width 0.3) (layer "F.Cu") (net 4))
 (segment (start 8.928 19.52) (end 8.128 20.32) (width 0.3) (layer "F.Cu") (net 4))
 (segment (start -1.228 1.228) (end 0 0) (width 0.3) (layer "F.Cu") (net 4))
 (segment (start 3.720999 49.059999) (end 8.382 49.059999) (width 0.3) (layer "F.Cu") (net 4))
 (segment (start 2.667 19.812) (end 2.159 20.32) (width 0.3) (layer "F.Cu") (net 4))
 (segment (start 15.24 21.463) (end 13.297 19.52) (width 0.3) (layer "F.Cu") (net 4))
 (segment (start 16.467999 19.092001) (end 15.24 20.32) (width 0.3) (layer "F.Cu") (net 4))
 (segment (start -1.228 24.088) (end 0 22.86) (width 0.3) (layer "F.Cu") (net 4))
 (segment (start 15.24 20.32) (end 15.24 21.463) (width 0.3) (layer "F.Cu") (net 4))
 (segment (start 8.128 21.2375) (end 8.128 20.32) (width 0.3) (layer "F.Cu") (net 4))
 (segment (start 4.496 21.59) (end 2.159 21.59) (width 0.3) (layer "F.Cu") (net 4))
 (segment (start 2.159 21.59) (end 0 21.59) (width 0.3) (layer "F.Cu") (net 4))
 (segment (start 4.496 1.27) (end 3.425 1.27) (width 0.3) (layer "F.Cu") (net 4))
 (segment (start 15.24 48.26) (end 9.181999 48.26) (width 0.3) (layer "F.Cu") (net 4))
 (segment (start -1.228 19.092) (end -1.228 1.228) (width 0.3) (layer "F.Cu") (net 4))
 (segment (start 0 21.59) (end 0 20.32) (width 0.3) (layer "F.Cu") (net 4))
 (segment (start 0 48.26) (end -1.228 47.032) (width 0.3) (layer "F.Cu") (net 4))
 (segment (start 9.181999 48.26) (end 8.382 49.059999) (width 0.3) (layer "F.Cu") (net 4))
 (segment (start 3.175 46.99) (end 2.921 47.244) (width 0.3) (layer "F.Cu") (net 4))
 (segment (start 16.467999 1.227999) (end 16.467999 19.092001) (width 0.3) (layer "F.Cu") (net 4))
 (segment (start 2.921 48.26) (end 3.720999 49.059999) (width 0.3) (layer "F.Cu") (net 4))
 (segment (start 16.468 47.032) (end 15.24 48.26) (width 0.3) (layer "F.Cu") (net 4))
 (segment (start 7.62 19.812) (end 2.667 19.812) (width 0.3) (layer "F.Cu") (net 4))
 (segment (start 14.097 -1.143) (end 15.24 0) (width 0.3) (layer "F.Cu") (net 4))
 (segment (start 8.128 20.32) (end 7.62 19.812) (width 0.3) (layer "F.Cu") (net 4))
 (segment (start 2.159 20.32) (end 2.159 21.59) (width 0.3) (layer "F.Cu") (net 4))
 (segment (start 15.24 22.86) (end 16.467999 24.087999) (width 0.3) (layer "F.Cu") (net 4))
 (segment (start 2.921 47.244) (end 2.921 48.26) (width 0.3) (layer "F.Cu") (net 4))
 (segment (start 0 20.32) (end -1.228 19.092) (width 0.3) (layer "F.Cu") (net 4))
 (segment (start 4.496001 46.99) (end 3.175 46.99) (width 0.3) (layer "F.Cu") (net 4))
 (segment (start 3.425 1.27) (end 3.175 1.52) (width 0.3) (layer "F.Cu") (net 4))
 (via (at 3.175 1.52) (size 0.8) (drill 0.4) (layers "F.Cu" "B.Cu") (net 4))
 (segment (start 1.655 0) (end 3.175 1.52) (width 0.3) (layer "B.Cu") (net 4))
 (segment (start 0 0) (end 1.655 0) (width 0.3) (layer "B.Cu") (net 4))
 (segment (start 4.496 1.77) (end 4.496 3.505) (width 0.2) (layer "F.Cu") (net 18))
 (segment (start 0 5.08) (end 4.445 5.08) (width 0.2) (layer "F.Cu") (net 18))
 (segment (start 4.445 3.556) (end 4.445 5.08) (width 0.2) (layer "F.Cu") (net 18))
 (segment (start 4.496 3.505) (end 4.445 3.556) (width 0.2) (layer "F.Cu") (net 18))
 (segment (start 4.445 5.08) (end 9.097 5.08) (width 0.2) (layer "F.Cu") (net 18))
 (segment (start 9.906 23.622) (end 9.906 21.4405) (width 0.2) (layer "F.Cu") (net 21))
 (segment (start 9.097 24.431) (end 9.906 23.622) (width 0.2) (layer "F.Cu") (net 21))
 (segment (start 10.2565 21.09) (end 10.744 21.09) (width 0.2) (layer "F.Cu") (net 21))
 (segment (start 0 25.4) (end 9.097 25.4) (width 0.2) (layer "F.Cu") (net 21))
 (segment (start 9.906 21.4405) (end 10.2565 21.09) (width 0.2) (layer "F.Cu") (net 21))
 (segment (start 9.097 25.4) (end 9.097 24.431) (width 0.2) (layer "F.Cu") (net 21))
 (segment (start 7.755 22.09) (end 7.747 22.098) (width 0.2) (layer "F.Cu") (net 14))
 (segment (start 0 15.24) (end 5.969 15.24) (width 0.2) (layer "F.Cu") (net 14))
 (segment (start 5.969 15.24) (end 9.097 15.24) (width 0.2) (layer "F.Cu") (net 14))
 (segment (start 9.068 22.09) (end 7.755 22.09) (width 0.2) (layer "F.Cu") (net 14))
 (via (at 5.969 15.24) (size 0.8) (drill 0.4) (layers "F.Cu" "B.Cu") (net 14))
 (via (at 7.747 22.098) (size 0.8) (drill 0.4) (layers "F.Cu" "B.Cu") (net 14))
 (segment (start 5.969 18.034) (end 5.969 15.24) (width 0.2) (layer "B.Cu") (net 14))
 (segment (start 7.747 19.812) (end 5.969 18.034) (width 0.2) (layer "B.Cu") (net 14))
 (segment (start 7.747 22.098) (end 7.747 19.812) (width 0.2) (layer "B.Cu") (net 14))
 (segment (start 9.068 20.511372) (end 9.201686 20.377686) (width 0.2) (layer "F.Cu") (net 12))
 (segment (start 0 12.7) (end 6.985 12.7) (width 0.2) (layer "F.Cu") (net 12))
 (segment (start 9.068 21.09) (end 9.068 20.511372) (width 0.2) (layer "F.Cu") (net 12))
 (segment (start 6.985 12.7) (end 9.097 12.7) (width 0.2) (layer "F.Cu") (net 12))
 (via (at 6.985 12.7) (size 0.8) (drill 0.4) (layers "F.Cu" "B.Cu") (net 12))
 (via (at 9.201686 20.377686) (size 0.8) (drill 0.4) (layers "F.Cu" "B.Cu") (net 12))
 (segment (start 8.255 18.161) (end 8.255 13.97) (width 0.2) (layer "B.Cu") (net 12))
 (segment (start 8.255 13.97) (end 6.985 12.7) (width 0.2) (layer "B.Cu") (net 12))
 (segment (start 9.201686 19.107686) (end 8.255 18.161) (width 0.2) (layer "B.Cu") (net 12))
 (segment (start 9.201686 20.377686) (end 9.201686 19.107686) (width 0.2) (layer "B.Cu") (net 12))
 (segment (start 9.769 17.77) (end 9.779 17.78) (width 0.2) (layer "F.Cu") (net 16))
 (segment (start 10.744 21.59) (end 11.557 21.59) (width 0.2) (layer "F.Cu") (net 16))
 (segment (start 9.097 17.77) (end 9.769 17.77) (width 0.2) (layer "F.Cu") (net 16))
 (segment (start 0 17.78) (end 9.779 17.78) (width 0.2) (layer "F.Cu") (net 16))
 (via (at 9.779 17.78) (size 0.8) (drill 0.4) (layers "F.Cu" "B.Cu") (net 16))
 (via (at 11.557 21.59) (size 0.8) (drill 0.4) (layers "F.Cu" "B.Cu") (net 16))
 (segment (start 11.557 19.558) (end 9.779 17.78) (width 0.2) (layer "B.Cu") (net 16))
 (segment (start 11.557 21.59) (end 11.557 19.558) (width 0.2) (layer "B.Cu") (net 16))
 (segment (start 4.445 30.48) (end 9.097 30.48) (width 0.2) (layer "F.Cu") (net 2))
 (segment (start 4.496 23.825) (end 4.445 23.876) (width 0.2) (layer "F.Cu") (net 2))
 (segment (start 0 30.48) (end 4.445 30.48) (width 0.2) (layer "F.Cu") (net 2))
 (segment (start 4.496 22.09) (end 4.496 23.825) (width 0.2) (layer "F.Cu") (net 2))
 (via (at 4.445 30.48) (size 0.8) (drill 0.4) (layers "F.Cu" "B.Cu") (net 2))
 (via (at 4.445 23.876) (size 0.8) (drill 0.4) (layers "F.Cu" "B.Cu") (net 2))
 (segment (start 4.445 30.48) (end 4.445 23.876) (width 0.2) (layer "B.Cu") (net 2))
 (segment (start 0 27.94) (end 3.429 27.94) (width 0.2) (layer "F.Cu") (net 29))
 (segment (start 4.496 21.09) (end 3.691 21.09) (width 0.2) (layer "F.Cu") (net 29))
 (segment (start 3.691 21.09) (end 3.429 20.828) (width 0.2) (layer "F.Cu") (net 29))
 (segment (start 3.429 27.94) (end 9.097 27.94) (width 0.2) (layer "F.Cu") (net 29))
 (via (at 3.429 27.94) (size 0.8) (drill 0.4) (layers "F.Cu" "B.Cu") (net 29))
 (via (at 3.429 20.828) (size 0.8) (drill 0.4) (layers "F.Cu" "B.Cu") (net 29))
 (segment (start 3.429 20.828) (end 3.429 27.94) (width 0.2) (layer "B.Cu") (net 29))
 (segment (start 0 33.02) (end 5.334 33.02) (width 0.2) (layer "F.Cu") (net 23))
 (segment (start 5.6845 21.59) (end 5.334 21.9405) (width 0.2) (layer "F.Cu") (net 23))
 (segment (start 5.334 21.9405) (end 5.334 24.511) (width 0.2) (layer "F.Cu") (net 23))
 (segment (start 5.334 33.02) (end 9.097 33.02) (width 0.2) (layer "F.Cu") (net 23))
 (segment (start 6.172 21.59) (end 5.6845 21.59) (width 0.2) (layer "F.Cu") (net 23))
 (via (at 5.334 24.511) (size 0.8) (drill 0.4) (layers "F.Cu" "B.Cu") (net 23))
 (via (at 5.334 33.02) (size 0.8) (drill 0.4) (layers "F.Cu" "B.Cu") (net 23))
 (segment (start 5.334 24.511) (end 5.334 33.02) (width 0.2) (layer "B.Cu") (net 23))
 (segment (start 6.985 35.56) (end 9.097 35.56) (width 0.2) (layer "F.Cu") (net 10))
 (segment (start 0 35.56) (end 6.985 35.56) (width 0.2) (layer "F.Cu") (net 10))
 (segment (start 6.723 21.09) (end 6.985 20.828) (width 0.2) (layer "F.Cu") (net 10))
 (segment (start 6.172 21.09) (end 6.723 21.09) (width 0.2) (layer "F.Cu") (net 10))
 (via (at 6.985 35.56) (size 0.8) (drill 0.4) (layers "F.Cu" "B.Cu") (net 10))
 (via (at 6.985 20.828) (size 0.8) (drill 0.4) (layers "F.Cu" "B.Cu") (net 10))
 (segment (start 6.985 20.828) (end 6.985 35.56) (width 0.2) (layer "B.Cu") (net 10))
 (segment (start 6.985 46.99) (end 7.239 47.244) (width 0.2) (layer "F.Cu") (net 7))
 (segment (start 9.097 43.18) (end 7.112 43.18) (width 0.2) (layer "F.Cu") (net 7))
 (segment (start 0 43.18) (end 7.112 43.18) (width 0.2) (layer "F.Cu") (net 7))
 (segment (start 6.171999 46.99) (end 6.985 46.99) (width 0.2) (layer "F.Cu") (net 7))
 (via (at 7.112 43.18) (size 0.8) (drill 0.4) (layers "F.Cu" "B.Cu") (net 7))
 (via (at 7.239 47.244) (size 0.8) (drill 0.4) (layers "F.Cu" "B.Cu") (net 7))
 (segment (start 7.239 47.244) (end 7.112 47.117) (width 0.2) (layer "B.Cu") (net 7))
 (segment (start 7.112 47.117) (end 7.112 43.18) (width 0.2) (layer "B.Cu") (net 7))
 (segment (start 7.104 46.49) (end 7.874 45.72) (width 0.2) (layer "F.Cu") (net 8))
 (segment (start 7.874 45.72) (end 9.097 45.72) (width 0.2) (layer "F.Cu") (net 8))
 (segment (start 5.596 46.49) (end 6.172 46.49) (width 0.2) (layer "F.Cu") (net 8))
 (segment (start 0 45.72) (end 4.826 45.72) (width 0.2) (layer "F.Cu") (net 8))
 (segment (start 4.826 45.72) (end 5.596 46.49) (width 0.2) (layer "F.Cu") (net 8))
 (segment (start 6.172 46.49) (end 7.104 46.49) (width 0.2) (layer "F.Cu") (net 8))
 (segment (start 2.54 38.1) (end 0 38.1) (width 0.2) (layer "F.Cu") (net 3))
 (segment (start 2.54 38.1) (end 9.097 38.1) (width 0.2) (layer "F.Cu") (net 3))
 (segment (start 2.548 46.49) (end 2.54 46.482) (width 0.2) (layer "F.Cu") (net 3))
 (segment (start 4.496 46.49) (end 2.548 46.49) (width 0.2) (layer "F.Cu") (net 3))
 (via (at 2.54 46.482) (size 0.8) (drill 0.4) (layers "F.Cu" "B.Cu") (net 3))
 (via (at 2.54 38.1) (size 0.8) (drill 0.4) (layers "F.Cu" "B.Cu") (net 3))
 (segment (start 2.54 46.482) (end 2.54 38.1) (width 0.2) (layer "B.Cu") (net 3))
 (segment (start 4.072 47.49) (end 3.81 47.752) (width 0.2) (layer "F.Cu") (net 5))
 (segment (start 3.81 40.64) (end 0 40.64) (width 0.2) (layer "F.Cu") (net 5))
 (segment (start 3.81 40.64) (end 9.097 40.64) (width 0.2) (layer "F.Cu") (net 5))
 (segment (start 4.496 47.49) (end 4.072 47.49) (width 0.2) (layer "F.Cu") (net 5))
 (via (at 3.81 47.752) (size 0.8) (drill 0.4) (layers "F.Cu" "B.Cu") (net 5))
 (via (at 3.81 40.64) (size 0.8) (drill 0.4) (layers "F.Cu" "B.Cu") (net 5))
 (segment (start 3.81 47.752) (end 3.81 40.64) (width 0.2) (layer "B.Cu") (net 5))
 (segment (start 10.922 17.77) (end 15.23 17.77) (width 0.2) (layer "F.Cu") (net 15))
 (segment (start 10.922 33.02) (end 15.24 33.02) (width 0.2) (layer "F.Cu") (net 22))
 (segment (start 15.24 5.08) (end 10.922 5.08) (width 0.2) (layer "F.Cu") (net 17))
 (segment (start 10.922 35.56) (end 15.24 35.56) (width 0.2) (layer "F.Cu") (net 9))
 (segment (start 10.922 45.72) (end 15.24 45.72) (width 0.2) (layer "F.Cu") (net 30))
 (segment (start 15.24 15.24) (end 10.922 15.24) (width 0.2) (layer "F.Cu") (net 13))
 (segment (start 10.922 40.64) (end 15.24 40.64) (width 0.2) (layer "F.Cu") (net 19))
 (segment (start 15.24 12.7) (end 10.922 12.7) (width 0.2) (layer "F.Cu") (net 11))
 (segment (start 10.922 38.1) (end 15.24 38.1) (width 0.2) (layer "F.Cu") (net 31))
 (segment (start 10.922 27.94) (end 15.24 27.94) (width 0.2) (layer "F.Cu") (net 32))
 (segment (start 10.922 43.18) (end 15.24 43.18) (width 0.2) (layer "F.Cu") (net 24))
 (segment (start 15.24 2.54) (end 10.922 2.54) (width 0.2) (layer "F.Cu") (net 25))
 (segment (start 15.24 7.62) (end 10.922 7.62) (width 0.2) (layer "F.Cu") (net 34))
 (segment (start 15.24 10.16) (end 10.932 10.16) (width 0.2) (layer "F.Cu") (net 33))
 (segment (start 10.922 30.48) (end 15.24 30.48) (width 0.2) (layer "F.Cu") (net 1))
 (segment (start 10.922 25.4) (end 15.24 25.4) (width 0.2) (layer "F.Cu") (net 20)))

